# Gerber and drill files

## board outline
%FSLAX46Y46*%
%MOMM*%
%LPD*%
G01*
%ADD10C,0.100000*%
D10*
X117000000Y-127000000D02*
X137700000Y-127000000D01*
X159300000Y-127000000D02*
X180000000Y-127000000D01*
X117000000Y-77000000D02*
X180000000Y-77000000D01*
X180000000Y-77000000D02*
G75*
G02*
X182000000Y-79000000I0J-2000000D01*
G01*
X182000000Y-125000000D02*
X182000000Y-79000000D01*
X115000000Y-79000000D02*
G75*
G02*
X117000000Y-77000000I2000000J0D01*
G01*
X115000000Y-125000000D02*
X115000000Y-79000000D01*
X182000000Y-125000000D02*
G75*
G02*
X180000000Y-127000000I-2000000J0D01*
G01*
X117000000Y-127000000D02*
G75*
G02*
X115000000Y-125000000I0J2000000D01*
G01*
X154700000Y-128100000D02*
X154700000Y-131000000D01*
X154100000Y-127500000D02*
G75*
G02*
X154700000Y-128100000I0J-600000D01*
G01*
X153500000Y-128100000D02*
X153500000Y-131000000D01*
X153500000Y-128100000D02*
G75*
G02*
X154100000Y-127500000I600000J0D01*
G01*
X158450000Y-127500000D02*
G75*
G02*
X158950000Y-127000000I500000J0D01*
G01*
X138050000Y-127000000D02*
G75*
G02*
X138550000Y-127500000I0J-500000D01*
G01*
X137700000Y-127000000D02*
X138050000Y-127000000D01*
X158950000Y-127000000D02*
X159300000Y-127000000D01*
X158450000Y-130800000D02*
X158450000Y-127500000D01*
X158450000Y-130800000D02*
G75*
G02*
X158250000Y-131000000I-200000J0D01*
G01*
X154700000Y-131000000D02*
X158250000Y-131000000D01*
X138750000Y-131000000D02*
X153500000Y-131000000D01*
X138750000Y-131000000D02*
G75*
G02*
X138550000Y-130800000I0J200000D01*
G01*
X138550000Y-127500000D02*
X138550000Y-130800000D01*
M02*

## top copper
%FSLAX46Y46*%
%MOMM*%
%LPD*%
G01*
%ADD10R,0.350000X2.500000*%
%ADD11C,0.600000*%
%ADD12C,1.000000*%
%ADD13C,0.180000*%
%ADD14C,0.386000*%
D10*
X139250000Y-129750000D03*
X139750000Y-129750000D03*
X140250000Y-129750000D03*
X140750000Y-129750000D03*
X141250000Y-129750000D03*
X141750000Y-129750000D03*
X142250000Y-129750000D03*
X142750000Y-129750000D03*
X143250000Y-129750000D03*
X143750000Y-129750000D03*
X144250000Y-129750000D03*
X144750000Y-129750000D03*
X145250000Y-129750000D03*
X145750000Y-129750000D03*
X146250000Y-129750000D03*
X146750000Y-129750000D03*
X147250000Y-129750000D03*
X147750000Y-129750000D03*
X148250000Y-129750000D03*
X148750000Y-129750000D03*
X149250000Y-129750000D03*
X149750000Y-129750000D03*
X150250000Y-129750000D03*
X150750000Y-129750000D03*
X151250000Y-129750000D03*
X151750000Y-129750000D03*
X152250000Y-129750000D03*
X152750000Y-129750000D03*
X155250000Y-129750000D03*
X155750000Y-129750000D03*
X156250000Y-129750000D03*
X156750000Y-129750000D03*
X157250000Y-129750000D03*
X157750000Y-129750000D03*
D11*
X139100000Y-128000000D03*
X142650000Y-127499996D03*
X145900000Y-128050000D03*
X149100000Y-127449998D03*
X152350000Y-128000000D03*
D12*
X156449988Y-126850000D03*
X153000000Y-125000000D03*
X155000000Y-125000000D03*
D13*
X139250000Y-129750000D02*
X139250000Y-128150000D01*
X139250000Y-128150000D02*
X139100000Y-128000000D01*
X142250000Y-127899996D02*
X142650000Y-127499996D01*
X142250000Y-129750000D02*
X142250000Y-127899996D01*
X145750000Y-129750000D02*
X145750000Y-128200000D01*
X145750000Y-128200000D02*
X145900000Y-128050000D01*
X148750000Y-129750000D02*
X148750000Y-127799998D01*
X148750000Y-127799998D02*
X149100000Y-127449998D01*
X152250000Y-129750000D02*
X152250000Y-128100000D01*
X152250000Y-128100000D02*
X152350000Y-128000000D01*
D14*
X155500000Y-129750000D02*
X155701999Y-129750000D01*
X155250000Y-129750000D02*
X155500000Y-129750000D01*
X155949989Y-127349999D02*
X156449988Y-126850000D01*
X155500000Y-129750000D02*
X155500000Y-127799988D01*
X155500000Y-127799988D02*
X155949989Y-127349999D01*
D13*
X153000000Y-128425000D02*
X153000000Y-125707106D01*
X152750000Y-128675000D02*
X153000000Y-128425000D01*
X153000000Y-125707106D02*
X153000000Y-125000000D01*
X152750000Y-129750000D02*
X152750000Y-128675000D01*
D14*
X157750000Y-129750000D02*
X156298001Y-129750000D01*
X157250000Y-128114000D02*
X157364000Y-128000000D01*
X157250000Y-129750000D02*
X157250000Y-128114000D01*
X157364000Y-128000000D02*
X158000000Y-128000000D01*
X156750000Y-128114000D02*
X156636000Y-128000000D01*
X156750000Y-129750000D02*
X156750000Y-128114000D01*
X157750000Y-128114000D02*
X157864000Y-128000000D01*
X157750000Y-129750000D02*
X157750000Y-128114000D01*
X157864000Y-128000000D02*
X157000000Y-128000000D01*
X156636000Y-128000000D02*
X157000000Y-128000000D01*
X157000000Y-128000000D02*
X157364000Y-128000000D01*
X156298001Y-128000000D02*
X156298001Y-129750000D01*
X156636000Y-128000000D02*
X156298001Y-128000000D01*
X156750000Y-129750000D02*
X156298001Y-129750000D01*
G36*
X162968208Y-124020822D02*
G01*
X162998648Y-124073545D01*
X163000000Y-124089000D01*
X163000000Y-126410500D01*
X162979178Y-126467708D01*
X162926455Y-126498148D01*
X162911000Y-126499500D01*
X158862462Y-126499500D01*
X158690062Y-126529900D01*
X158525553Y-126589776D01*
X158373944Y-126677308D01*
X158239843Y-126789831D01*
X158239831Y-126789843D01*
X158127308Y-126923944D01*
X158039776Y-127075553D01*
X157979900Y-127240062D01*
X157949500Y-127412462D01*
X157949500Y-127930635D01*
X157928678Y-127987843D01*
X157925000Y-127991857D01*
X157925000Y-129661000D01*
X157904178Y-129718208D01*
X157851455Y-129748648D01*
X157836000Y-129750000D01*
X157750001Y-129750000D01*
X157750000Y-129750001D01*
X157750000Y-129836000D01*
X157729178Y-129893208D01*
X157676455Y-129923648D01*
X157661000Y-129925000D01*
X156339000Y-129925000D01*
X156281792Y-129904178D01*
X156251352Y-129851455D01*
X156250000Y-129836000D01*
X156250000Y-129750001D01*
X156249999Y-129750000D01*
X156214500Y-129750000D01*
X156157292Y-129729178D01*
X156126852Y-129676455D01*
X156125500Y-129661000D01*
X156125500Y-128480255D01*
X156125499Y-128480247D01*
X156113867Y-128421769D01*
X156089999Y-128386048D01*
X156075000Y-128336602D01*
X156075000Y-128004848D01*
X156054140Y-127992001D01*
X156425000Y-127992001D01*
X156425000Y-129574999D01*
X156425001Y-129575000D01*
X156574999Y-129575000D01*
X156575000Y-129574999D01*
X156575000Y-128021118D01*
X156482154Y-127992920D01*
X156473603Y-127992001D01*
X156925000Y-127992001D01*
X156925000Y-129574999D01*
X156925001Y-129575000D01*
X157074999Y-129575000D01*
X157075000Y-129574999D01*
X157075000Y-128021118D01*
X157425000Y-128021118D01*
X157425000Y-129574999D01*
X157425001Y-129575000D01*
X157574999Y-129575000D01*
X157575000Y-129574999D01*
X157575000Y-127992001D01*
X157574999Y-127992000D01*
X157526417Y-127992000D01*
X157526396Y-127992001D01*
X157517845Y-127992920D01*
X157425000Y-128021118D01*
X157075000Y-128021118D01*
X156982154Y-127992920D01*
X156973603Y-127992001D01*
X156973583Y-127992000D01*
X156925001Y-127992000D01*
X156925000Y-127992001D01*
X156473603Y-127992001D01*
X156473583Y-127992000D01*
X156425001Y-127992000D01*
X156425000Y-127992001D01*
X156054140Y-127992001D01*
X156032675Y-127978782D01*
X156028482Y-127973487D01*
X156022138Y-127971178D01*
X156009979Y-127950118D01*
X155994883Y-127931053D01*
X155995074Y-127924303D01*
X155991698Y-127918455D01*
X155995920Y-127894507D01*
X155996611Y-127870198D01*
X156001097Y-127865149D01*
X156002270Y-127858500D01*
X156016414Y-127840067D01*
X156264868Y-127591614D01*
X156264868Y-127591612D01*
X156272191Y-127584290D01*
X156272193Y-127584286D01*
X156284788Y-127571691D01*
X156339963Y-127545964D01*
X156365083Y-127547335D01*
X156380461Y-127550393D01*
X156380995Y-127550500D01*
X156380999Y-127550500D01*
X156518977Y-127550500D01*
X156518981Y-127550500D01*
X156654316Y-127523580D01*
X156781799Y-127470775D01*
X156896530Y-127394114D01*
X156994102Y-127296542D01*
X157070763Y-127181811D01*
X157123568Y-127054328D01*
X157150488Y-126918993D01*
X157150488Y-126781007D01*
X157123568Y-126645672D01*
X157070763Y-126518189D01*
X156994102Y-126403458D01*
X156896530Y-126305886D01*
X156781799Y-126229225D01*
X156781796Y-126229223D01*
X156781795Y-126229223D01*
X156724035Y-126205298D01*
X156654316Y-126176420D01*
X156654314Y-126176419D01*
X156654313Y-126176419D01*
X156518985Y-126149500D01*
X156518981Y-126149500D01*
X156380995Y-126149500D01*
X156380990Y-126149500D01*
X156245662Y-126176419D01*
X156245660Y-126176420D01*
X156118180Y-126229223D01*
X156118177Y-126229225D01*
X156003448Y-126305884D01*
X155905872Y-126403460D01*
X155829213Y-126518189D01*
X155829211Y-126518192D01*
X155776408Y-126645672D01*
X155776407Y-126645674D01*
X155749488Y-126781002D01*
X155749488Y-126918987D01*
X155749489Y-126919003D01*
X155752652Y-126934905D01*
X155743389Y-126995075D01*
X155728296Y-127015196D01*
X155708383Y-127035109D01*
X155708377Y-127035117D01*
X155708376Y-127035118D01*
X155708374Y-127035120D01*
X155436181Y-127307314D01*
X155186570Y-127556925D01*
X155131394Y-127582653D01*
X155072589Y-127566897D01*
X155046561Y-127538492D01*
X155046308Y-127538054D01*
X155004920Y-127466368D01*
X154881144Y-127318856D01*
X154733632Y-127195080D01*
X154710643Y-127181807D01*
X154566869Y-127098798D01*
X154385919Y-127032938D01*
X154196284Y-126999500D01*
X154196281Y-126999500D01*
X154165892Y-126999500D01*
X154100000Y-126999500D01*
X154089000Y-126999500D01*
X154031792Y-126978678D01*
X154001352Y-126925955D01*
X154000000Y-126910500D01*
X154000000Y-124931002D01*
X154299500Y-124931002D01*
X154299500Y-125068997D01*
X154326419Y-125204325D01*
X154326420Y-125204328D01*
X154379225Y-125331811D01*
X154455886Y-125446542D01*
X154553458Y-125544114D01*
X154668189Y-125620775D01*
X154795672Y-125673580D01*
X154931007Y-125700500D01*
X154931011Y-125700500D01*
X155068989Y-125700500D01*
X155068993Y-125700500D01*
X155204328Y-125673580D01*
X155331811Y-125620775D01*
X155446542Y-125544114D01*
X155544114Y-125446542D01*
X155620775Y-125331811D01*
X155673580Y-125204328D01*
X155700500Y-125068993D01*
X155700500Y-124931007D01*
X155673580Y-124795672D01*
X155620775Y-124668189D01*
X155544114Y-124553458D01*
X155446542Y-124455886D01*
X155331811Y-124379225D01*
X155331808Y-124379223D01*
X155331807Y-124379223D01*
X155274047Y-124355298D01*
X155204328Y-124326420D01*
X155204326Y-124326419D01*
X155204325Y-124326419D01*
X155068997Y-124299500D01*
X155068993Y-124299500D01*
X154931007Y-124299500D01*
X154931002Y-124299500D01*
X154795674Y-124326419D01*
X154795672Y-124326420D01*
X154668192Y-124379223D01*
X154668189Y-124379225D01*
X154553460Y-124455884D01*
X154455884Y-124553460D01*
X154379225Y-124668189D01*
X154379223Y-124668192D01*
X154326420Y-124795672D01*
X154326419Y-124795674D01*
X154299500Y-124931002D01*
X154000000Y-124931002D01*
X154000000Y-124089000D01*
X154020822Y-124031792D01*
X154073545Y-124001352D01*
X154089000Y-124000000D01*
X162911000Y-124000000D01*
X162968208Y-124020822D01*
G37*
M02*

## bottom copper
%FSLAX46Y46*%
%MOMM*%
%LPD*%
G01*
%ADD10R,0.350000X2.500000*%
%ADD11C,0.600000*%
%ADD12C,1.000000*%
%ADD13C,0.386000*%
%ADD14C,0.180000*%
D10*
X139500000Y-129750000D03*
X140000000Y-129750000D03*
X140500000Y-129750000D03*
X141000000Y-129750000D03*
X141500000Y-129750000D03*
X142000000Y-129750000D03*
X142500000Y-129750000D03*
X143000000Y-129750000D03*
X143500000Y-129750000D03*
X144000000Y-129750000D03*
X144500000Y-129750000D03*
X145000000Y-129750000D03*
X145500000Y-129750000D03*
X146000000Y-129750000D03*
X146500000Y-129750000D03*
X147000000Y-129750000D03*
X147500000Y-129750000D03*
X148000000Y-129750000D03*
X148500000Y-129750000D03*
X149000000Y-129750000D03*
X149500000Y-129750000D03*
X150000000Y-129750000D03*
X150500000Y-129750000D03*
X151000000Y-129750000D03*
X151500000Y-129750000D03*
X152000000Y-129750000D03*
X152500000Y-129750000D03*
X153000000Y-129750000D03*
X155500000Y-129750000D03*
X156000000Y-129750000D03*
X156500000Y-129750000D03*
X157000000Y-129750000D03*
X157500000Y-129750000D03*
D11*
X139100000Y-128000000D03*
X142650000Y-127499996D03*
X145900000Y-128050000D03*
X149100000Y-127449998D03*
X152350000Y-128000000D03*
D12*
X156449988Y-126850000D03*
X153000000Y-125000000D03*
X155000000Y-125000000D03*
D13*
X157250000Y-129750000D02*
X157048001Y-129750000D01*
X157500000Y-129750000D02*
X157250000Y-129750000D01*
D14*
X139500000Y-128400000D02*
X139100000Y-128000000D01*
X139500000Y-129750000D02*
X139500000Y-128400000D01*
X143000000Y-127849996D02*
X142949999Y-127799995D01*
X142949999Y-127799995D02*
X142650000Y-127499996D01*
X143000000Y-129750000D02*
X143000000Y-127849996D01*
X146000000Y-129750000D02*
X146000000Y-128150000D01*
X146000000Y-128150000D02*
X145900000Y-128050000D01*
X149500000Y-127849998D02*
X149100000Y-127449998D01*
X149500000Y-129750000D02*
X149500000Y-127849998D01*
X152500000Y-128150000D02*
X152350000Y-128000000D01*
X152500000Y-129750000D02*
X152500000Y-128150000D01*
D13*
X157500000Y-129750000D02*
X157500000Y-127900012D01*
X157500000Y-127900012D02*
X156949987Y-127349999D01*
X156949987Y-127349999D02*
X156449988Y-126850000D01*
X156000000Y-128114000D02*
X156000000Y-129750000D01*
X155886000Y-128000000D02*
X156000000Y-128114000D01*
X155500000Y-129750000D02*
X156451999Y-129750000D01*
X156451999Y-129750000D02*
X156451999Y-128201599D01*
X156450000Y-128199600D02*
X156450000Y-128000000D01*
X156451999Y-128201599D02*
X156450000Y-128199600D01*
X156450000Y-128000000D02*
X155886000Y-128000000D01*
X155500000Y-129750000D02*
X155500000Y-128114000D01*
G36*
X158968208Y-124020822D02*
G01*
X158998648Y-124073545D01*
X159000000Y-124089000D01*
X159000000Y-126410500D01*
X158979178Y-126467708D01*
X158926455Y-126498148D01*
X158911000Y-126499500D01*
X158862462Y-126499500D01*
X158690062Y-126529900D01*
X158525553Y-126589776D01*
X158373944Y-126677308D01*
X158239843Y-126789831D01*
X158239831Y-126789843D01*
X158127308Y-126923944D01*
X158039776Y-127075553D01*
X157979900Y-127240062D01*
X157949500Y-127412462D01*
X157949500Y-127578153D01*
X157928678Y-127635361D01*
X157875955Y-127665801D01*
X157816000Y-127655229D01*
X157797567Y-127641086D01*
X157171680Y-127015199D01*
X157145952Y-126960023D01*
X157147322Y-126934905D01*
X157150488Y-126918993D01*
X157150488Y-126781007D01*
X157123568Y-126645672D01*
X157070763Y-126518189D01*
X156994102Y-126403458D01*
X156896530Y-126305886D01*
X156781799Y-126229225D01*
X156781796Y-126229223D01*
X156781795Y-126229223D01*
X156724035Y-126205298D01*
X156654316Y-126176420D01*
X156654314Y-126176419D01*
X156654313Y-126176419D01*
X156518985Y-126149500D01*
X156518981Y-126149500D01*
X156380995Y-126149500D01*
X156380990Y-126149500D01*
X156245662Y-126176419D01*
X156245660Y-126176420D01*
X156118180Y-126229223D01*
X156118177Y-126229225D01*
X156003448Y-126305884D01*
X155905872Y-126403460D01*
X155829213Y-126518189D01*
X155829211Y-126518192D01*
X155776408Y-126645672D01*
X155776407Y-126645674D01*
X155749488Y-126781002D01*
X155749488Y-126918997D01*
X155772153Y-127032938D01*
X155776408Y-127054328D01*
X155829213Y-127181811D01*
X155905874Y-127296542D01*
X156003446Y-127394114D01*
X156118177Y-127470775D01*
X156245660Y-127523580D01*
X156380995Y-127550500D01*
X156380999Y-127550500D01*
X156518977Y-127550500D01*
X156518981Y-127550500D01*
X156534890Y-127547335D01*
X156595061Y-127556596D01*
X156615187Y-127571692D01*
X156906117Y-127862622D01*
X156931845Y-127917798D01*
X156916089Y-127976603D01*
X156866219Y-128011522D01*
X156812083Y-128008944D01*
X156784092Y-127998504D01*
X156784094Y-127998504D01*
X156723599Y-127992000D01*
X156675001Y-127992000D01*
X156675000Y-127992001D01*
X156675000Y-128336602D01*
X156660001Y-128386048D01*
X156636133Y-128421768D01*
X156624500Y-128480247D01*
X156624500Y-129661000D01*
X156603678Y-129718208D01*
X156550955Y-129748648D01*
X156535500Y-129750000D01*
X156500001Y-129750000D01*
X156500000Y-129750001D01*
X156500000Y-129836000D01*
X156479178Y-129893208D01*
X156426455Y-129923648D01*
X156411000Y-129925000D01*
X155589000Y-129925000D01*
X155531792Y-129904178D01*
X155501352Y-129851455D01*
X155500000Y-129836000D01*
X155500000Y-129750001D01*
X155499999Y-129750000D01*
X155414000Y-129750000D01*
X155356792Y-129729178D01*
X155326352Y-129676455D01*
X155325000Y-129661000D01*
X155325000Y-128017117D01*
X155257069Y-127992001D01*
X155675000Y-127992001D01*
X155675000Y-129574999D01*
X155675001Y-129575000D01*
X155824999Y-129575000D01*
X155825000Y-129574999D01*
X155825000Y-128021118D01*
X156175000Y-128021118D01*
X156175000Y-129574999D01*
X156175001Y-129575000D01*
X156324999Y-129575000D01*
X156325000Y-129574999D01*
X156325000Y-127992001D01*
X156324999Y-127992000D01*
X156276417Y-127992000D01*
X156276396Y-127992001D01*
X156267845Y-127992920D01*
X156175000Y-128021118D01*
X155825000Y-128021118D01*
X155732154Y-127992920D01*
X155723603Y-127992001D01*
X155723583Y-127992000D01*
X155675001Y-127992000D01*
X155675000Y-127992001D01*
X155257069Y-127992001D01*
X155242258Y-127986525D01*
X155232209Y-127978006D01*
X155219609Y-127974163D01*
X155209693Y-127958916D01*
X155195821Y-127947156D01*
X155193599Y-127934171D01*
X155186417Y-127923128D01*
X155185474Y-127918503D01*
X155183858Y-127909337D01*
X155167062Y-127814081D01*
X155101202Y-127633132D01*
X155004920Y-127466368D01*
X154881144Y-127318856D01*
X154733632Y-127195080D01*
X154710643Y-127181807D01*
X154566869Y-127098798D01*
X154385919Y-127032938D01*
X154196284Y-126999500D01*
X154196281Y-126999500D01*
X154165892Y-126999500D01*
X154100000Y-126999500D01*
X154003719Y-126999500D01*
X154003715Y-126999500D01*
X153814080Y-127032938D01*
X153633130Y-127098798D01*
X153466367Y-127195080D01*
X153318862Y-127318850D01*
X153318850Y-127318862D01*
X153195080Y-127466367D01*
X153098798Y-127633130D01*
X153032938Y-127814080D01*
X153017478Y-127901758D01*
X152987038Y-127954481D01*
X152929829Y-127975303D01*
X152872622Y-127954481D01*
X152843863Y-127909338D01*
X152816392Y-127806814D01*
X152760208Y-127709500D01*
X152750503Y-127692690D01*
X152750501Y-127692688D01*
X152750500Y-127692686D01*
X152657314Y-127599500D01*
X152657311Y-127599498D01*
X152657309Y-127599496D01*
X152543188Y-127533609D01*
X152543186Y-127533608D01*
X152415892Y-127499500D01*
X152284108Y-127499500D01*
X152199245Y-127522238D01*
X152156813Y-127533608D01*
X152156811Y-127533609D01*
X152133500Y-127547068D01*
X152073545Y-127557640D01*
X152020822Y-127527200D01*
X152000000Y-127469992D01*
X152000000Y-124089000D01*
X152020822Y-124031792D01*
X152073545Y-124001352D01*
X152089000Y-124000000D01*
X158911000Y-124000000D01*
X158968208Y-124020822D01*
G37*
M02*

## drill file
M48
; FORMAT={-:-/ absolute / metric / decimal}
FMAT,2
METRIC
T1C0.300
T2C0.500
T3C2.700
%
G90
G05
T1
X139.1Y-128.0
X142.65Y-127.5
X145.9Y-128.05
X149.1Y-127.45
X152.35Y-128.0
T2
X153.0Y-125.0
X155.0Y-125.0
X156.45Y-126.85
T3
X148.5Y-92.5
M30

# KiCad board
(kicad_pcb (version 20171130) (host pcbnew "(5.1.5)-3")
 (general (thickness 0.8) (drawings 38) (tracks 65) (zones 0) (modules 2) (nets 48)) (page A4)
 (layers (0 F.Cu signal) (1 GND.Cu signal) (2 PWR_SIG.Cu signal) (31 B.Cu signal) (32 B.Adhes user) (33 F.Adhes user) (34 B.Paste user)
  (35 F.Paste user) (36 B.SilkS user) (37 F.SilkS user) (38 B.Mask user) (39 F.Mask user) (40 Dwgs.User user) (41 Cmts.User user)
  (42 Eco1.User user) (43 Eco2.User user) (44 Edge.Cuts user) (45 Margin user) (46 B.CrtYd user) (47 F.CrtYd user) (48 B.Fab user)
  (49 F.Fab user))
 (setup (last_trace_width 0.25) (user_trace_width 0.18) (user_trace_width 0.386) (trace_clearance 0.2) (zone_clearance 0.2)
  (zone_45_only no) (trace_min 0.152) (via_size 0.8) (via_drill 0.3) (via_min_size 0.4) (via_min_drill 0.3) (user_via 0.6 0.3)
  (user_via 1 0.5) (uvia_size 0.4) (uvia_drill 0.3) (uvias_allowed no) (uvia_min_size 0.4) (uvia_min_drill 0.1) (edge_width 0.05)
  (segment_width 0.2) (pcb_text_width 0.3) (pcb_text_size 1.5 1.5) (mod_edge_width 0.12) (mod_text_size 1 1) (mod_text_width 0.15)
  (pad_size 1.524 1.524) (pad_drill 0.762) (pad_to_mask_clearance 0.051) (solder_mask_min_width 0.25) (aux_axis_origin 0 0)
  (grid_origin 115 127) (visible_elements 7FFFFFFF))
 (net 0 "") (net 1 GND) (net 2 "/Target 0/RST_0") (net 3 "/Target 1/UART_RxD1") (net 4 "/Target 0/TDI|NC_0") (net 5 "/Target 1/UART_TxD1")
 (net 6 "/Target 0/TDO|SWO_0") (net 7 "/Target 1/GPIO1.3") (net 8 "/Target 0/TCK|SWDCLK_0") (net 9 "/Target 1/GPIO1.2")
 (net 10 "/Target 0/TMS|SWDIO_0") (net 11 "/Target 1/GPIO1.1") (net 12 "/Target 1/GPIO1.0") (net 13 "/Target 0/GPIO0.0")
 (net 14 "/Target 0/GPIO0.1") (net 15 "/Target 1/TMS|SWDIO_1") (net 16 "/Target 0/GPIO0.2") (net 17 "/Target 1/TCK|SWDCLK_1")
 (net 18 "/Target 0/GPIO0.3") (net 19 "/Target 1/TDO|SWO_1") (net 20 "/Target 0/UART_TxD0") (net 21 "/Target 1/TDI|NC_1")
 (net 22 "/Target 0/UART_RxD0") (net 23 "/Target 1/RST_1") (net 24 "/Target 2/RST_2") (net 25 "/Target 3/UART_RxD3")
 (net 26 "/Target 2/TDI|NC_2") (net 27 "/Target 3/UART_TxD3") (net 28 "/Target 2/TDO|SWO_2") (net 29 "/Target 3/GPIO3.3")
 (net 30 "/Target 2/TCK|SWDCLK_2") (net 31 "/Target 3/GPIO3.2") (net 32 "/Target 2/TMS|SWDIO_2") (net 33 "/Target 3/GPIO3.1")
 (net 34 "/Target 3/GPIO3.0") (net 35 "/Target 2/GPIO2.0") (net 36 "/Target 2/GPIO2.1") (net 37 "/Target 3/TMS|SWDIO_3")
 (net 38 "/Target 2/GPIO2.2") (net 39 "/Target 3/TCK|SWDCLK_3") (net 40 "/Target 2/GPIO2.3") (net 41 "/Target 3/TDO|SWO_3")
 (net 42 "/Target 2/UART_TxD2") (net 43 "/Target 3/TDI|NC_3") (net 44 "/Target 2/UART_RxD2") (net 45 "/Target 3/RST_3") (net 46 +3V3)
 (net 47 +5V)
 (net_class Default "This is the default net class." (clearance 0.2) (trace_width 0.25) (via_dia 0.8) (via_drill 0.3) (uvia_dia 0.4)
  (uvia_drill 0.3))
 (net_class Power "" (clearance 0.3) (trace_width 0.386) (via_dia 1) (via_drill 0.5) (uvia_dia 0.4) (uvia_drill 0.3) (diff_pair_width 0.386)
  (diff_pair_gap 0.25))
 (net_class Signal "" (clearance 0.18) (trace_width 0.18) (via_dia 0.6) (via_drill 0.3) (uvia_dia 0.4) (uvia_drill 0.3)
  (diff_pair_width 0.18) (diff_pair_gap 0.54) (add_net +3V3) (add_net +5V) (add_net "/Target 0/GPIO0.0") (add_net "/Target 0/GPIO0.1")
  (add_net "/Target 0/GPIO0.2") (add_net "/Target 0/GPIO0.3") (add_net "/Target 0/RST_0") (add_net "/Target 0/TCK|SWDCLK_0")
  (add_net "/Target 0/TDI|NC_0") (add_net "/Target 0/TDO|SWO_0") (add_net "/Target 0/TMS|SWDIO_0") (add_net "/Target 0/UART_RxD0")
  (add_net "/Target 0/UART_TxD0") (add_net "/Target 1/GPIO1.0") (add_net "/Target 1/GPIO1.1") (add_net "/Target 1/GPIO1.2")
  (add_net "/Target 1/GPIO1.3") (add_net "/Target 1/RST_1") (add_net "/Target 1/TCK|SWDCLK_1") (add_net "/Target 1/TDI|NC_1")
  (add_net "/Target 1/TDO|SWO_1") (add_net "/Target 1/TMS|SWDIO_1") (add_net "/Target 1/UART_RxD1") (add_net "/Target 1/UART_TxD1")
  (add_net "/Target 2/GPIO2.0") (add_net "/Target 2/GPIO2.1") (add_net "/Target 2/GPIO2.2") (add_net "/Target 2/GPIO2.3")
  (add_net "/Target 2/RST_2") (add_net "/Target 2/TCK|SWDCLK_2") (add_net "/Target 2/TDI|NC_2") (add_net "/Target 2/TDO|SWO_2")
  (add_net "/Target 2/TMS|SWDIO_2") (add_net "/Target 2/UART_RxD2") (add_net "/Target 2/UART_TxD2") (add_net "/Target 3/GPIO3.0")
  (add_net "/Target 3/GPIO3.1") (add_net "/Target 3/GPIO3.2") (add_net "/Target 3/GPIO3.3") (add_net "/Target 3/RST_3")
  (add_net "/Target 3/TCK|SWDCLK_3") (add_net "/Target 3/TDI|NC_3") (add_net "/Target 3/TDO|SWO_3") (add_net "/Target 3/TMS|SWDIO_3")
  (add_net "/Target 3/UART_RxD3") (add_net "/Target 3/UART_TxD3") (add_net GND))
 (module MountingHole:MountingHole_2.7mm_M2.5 (layer F.Cu) (at 148.5 92.5)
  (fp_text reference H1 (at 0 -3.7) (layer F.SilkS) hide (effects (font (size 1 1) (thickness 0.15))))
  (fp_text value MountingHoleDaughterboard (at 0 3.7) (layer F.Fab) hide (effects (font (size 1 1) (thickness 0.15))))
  (pad 1 np_thru_hole circle (at 0 0) (size 2.7 2.7) (drill 2.7) (layers *.Cu *.Mask)))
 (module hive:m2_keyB (layer F.Cu) (at 148.5 131)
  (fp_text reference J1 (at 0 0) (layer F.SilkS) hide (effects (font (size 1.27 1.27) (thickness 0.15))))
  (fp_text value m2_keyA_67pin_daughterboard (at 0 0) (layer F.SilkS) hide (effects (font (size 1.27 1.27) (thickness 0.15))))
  (fp_line (start 6.2 -2.9) (end 6.2 0) (layer Edge.Cuts) (width 0.1))
  (fp_arc (start 5.6 -2.9) (end 5.6 -3.5) (angle 90) (layer Edge.Cuts) (width 0.1))
  (fp_line (start 5 -2.9) (end 5 0) (layer Edge.Cuts) (width 0.1))
  (fp_arc (start 5.6 -2.9) (end 5.6 -3.5) (angle -90) (layer Edge.Cuts) (width 0.1))
  (fp_arc (start 10.45 -3.5) (end 9.95 -3.5) (angle 90) (layer Edge.Cuts) (width 0.1))
  (fp_arc (start -10.45 -3.5) (end -10.45 -4) (angle 90) (layer Edge.Cuts) (width 0.1))
  (fp_line (start -10.8 -4) (end -10.45 -4) (layer Edge.Cuts) (width 0.1))
  (fp_line (start 10.45 -4) (end 10.8 -4) (layer Edge.Cuts) (width 0.1))
  (fp_line (start 9.95 -0.2) (end 9.95 -3.5) (layer Edge.Cuts) (width 0.1))
  (fp_arc (start 9.75 -0.2) (end 9.75 0) (angle -90) (layer Edge.Cuts) (width 0.1))
  (fp_line (start 6.2 0) (end 9.75 0) (layer Edge.Cuts) (width 0.1))
  (fp_line (start -9.75 0) (end 5 0) (layer Edge.Cuts) (width 0.1))
  (fp_arc (start -9.75 -0.2) (end -9.95 -0.2) (angle -90) (layer Edge.Cuts) (width 0.1))
  (fp_line (start -9.95 -3.5) (end -9.95 -0.2) (layer Edge.Cuts) (width 0.1))
  (pad 75 smd rect (at -9.25 -1.25) (size 0.35 2.5) (layers F.Cu F.Paste F.Mask) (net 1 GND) (solder_mask_margin 0.1016))
  (pad 74 smd rect (at -9 -1.25) (size 0.35 2.5) (layers B.Cu B.Paste B.Mask) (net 1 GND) (solder_mask_margin 0.1016))
  (pad 73 smd rect (at -8.75 -1.25) (size 0.35 2.5) (layers F.Cu F.Paste F.Mask) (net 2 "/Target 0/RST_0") (solder_mask_margin 0.1016))
  (pad 72 smd rect (at -8.5 -1.25) (size 0.35 2.5) (layers B.Cu B.Paste B.Mask) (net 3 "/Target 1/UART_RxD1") (solder_mask_margin 0.1016))
  (pad 71 smd rect (at -8.25 -1.25) (size 0.35 2.5) (layers F.Cu F.Paste F.Mask) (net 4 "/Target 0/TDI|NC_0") (solder_mask_margin 0.1016))
  (pad 70 smd rect (at -8 -1.25) (size 0.35 2.5) (layers B.Cu B.Paste B.Mask) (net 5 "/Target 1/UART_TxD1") (solder_mask_margin 0.1016))
  (pad 69 smd rect (at -7.75 -1.25) (size 0.35 2.5) (layers F.Cu F.Paste F.Mask) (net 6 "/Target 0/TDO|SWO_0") (solder_mask_margin 0.1016))
  (pad 68 smd rect (at -7.5 -1.25) (size 0.35 2.5) (layers B.Cu B.Paste B.Mask) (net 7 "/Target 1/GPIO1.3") (solder_mask_margin 0.1016))
  (pad 67 smd rect (at -7.25 -1.25) (size 0.35 2.5) (layers F.Cu F.Paste F.Mask) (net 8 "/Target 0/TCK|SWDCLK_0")
   (solder_mask_margin 0.1016))
  (pad 66 smd rect (at -7 -1.25) (size 0.35 2.5) (layers B.Cu B.Paste B.Mask) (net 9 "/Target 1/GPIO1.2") (solder_mask_margin 0.1016))
  (pad 65 smd rect (at -6.75 -1.25) (size 0.35 2.5) (layers F.Cu F.Paste F.Mask) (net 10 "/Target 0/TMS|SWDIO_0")
   (solder_mask_margin 0.1016))
  (pad 64 smd rect (at -6.5 -1.25) (size 0.35 2.5) (layers B.Cu B.Paste B.Mask) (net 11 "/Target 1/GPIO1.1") (solder_mask_margin 0.1016))
  (pad 63 smd rect (at -6.25 -1.25) (size 0.35 2.5) (layers F.Cu F.Paste F.Mask) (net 1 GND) (solder_mask_margin 0.1016))
  (pad 62 smd rect (at -6 -1.25) (size 0.35 2.5) (layers B.Cu B.Paste B.Mask) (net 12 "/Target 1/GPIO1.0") (solder_mask_margin 0.1016))
  (pad 61 smd rect (at -5.75 -1.25) (size 0.35 2.5) (layers F.Cu F.Paste F.Mask) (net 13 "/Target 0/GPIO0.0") (solder_mask_margin 0.1016))
  (pad 60 smd rect (at -5.5 -1.25) (size 0.35 2.5) (layers B.Cu B.Paste B.Mask) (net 1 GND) (solder_mask_margin 0.1016))
  (pad 59 smd rect (at -5.25 -1.25) (size 0.35 2.5) (layers F.Cu F.Paste F.Mask) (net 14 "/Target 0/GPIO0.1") (solder_mask_margin 0.1016))
  (pad 58 smd rect (at -5 -1.25) (size 0.35 2.5) (layers B.Cu B.Paste B.Mask) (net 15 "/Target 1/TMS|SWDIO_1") (solder_mask_margin 0.1016))
  (pad 57 smd rect (at -4.75 -1.25) (size 0.35 2.5) (layers F.Cu F.Paste F.Mask) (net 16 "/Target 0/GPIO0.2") (solder_mask_margin 0.1016))
  (pad 56 smd rect (at -4.5 -1.25) (size 0.35 2.5) (layers B.Cu B.Paste B.Mask) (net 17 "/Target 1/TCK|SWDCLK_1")
   (solder_mask_margin 0.1016))
  (pad 55 smd rect (at -4.25 -1.25) (size 0.35 2.5) (layers F.Cu F.Paste F.Mask) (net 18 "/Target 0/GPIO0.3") (solder_mask_margin 0.1016))
  (pad 54 smd rect (at -4 -1.25) (size 0.35 2.5) (layers B.Cu B.Paste B.Mask) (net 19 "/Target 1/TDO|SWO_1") (solder_mask_margin 0.1016))
  (pad 53 smd rect (at -3.75 -1.25) (size 0.35 2.5) (layers F.Cu F.Paste F.Mask) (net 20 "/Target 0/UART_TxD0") (solder_mask_margin 0.1016))
  (pad 52 smd rect (at -3.5 -1.25) (size 0.35 2.5) (layers B.Cu B.Paste B.Mask) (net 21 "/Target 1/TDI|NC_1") (solder_mask_margin 0.1016))
  (pad 51 smd rect (at -3.25 -1.25) (size 0.35 2.5) (layers F.Cu F.Paste F.Mask) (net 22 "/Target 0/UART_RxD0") (solder_mask_margin 0.1016))
  (pad 50 smd rect (at -3 -1.25) (size 0.35 2.5) (layers B.Cu B.Paste B.Mask) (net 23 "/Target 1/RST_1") (solder_mask_margin 0.1016))
  (pad 49 smd rect (at -2.75 -1.25) (size 0.35 2.5) (layers F.Cu F.Paste F.Mask) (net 1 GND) (solder_mask_margin 0.1016))
  (pad 48 smd rect (at -2.5 -1.25) (size 0.35 2.5) (layers B.Cu B.Paste B.Mask) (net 1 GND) (solder_mask_margin 0.1016))
  (pad 47 smd rect (at -2.25 -1.25) (size 0.35 2.5) (layers F.Cu F.Paste F.Mask) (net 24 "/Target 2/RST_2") (solder_mask_margin 0.1016))
  (pad 46 smd rect (at -2 -1.25) (size 0.35 2.5) (layers B.Cu B.Paste B.Mask) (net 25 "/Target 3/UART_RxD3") (solder_mask_margin 0.1016))
  (pad 45 smd rect (at -1.75 -1.25) (size 0.35 2.5) (layers F.Cu F.Paste F.Mask) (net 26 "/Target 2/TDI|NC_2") (solder_mask_margin 0.1016))
  (pad 44 smd rect (at -1.5 -1.25) (size 0.35 2.5) (layers B.Cu B.Paste B.Mask) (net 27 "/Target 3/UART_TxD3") (solder_mask_margin 0.1016))
  (pad 43 smd rect (at -1.25 -1.25) (size 0.35 2.5) (layers F.Cu F.Paste F.Mask) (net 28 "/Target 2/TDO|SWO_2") (solder_mask_margin 0.1016))
  (pad 42 smd rect (at -1 -1.25) (size 0.35 2.5) (layers B.Cu B.Paste B.Mask) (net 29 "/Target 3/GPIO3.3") (solder_mask_margin 0.1016))
  (pad 41 smd rect (at -0.75 -1.25) (size 0.35 2.5) (layers F.Cu F.Paste F.Mask) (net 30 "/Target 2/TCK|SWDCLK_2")
   (solder_mask_margin 0.1016))
  (pad 40 smd rect (at -0.5 -1.25) (size 0.35 2.5) (layers B.Cu B.Paste B.Mask) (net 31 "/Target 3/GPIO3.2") (solder_mask_margin 0.1016))
  (pad 39 smd rect (at -0.25 -1.25) (size 0.35 2.5) (layers F.Cu F.Paste F.Mask) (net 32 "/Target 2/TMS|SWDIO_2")
   (solder_mask_margin 0.1016))
  (pad 38 smd rect (at 0 -1.25) (size 0.35 2.5) (layers B.Cu B.Paste B.Mask) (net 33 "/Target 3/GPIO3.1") (solder_mask_margin 0.1016))
  (pad 37 smd rect (at 0.25 -1.25) (size 0.35 2.5) (layers F.Cu F.Paste F.Mask) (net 1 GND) (solder_mask_margin 0.1016))
  (pad 36 smd rect (at 0.5 -1.25) (size 0.35 2.5) (layers B.Cu B.Paste B.Mask) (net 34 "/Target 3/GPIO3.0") (solder_mask_margin 0.1016))
  (pad 35 smd rect (at 0.75 -1.25) (size 0.35 2.5) (layers F.Cu F.Paste F.Mask) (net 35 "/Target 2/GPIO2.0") (solder_mask_margin 0.1016))
  (pad 34 smd rect (at 1 -1.25) (size 0.35 2.5) (layers B.Cu B.Paste B.Mask) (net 1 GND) (solder_mask_margin 0.1016))
  (pad 33 smd rect (at 1.25 -1.25) (size 0.35 2.5) (layers F.Cu F.Paste F.Mask) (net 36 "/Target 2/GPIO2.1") (solder_mask_margin 0.1016))
  (pad 32 smd rect (at 1.5 -1.25) (size 0.35 2.5) (layers B.Cu B.Paste B.Mask) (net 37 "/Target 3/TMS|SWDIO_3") (solder_mask_margin 0.1016))
  (pad 31 smd rect (at 1.75 -1.25) (size 0.35 2.5) (layers F.Cu F.Paste F.Mask) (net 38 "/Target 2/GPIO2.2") (solder_mask_margin 0.1016))
  (pad 30 smd rect (at 2 -1.25) (size 0.35 2.5) (layers B.Cu B.Paste B.Mask) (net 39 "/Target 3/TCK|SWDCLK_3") (solder_mask_margin 0.1016))
  (pad 29 smd rect (at 2.25 -1.25) (size 0.35 2.5) (layers F.Cu F.Paste F.Mask) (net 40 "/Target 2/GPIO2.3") (solder_mask_margin 0.1016))
  (pad 28 smd rect (at 2.5 -1.25) (size 0.35 2.5) (layers B.Cu B.Paste B.Mask) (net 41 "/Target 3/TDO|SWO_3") (solder_mask_margin 0.1016))
  (pad 27 smd rect (at 2.75 -1.25) (size 0.35 2.5) (layers F.Cu F.Paste F.Mask) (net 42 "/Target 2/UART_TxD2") (solder_mask_margin 0.1016))
  (pad 26 smd rect (at 3 -1.25) (size 0.35 2.5) (layers B.Cu B.Paste B.Mask) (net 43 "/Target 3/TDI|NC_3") (solder_mask_margin 0.1016))
  (pad 25 smd rect (at 3.25 -1.25) (size 0.35 2.5) (layers F.Cu F.Paste F.Mask) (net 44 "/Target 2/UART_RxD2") (solder_mask_margin 0.1016))
  (pad 24 smd rect (at 3.5 -1.25) (size 0.35 2.5) (layers B.Cu B.Paste B.Mask) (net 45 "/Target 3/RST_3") (solder_mask_margin 0.1016))
  (pad 23 smd rect (at 3.75 -1.25) (size 0.35 2.5) (layers F.Cu F.Paste F.Mask) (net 1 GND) (solder_mask_margin 0.1016))
  (pad 22 smd rect (at 4 -1.25) (size 0.35 2.5) (layers B.Cu B.Paste B.Mask) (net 1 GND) (solder_mask_margin 0.1016))
  (pad 21 smd rect (at 4.25 -1.25) (size 0.35 2.5) (layers F.Cu F.Paste F.Mask) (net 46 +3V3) (solder_mask_margin 0.1016))
  (pad 20 smd rect (at 4.5 -1.25) (size 0.35 2.5) (layers B.Cu B.Paste B.Mask) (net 46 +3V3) (solder_mask_margin 0.1016))
  (pad 11 smd rect (at 6.75 -1.25) (size 0.35 2.5) (layers F.Cu F.Paste F.Mask) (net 1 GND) (solder_mask_margin 0.1016))
  (pad 10 smd rect (at 7 -1.25) (size 0.35 2.5) (layers B.Cu B.Paste B.Mask) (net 46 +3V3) (solder_mask_margin 0.1016))
  (pad 9 smd rect (at 7.25 -1.25) (size 0.35 2.5) (layers F.Cu F.Paste F.Mask) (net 1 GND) (solder_mask_margin 0.1016))
  (pad 8 smd rect (at 7.5 -1.25) (size 0.35 2.5) (layers B.Cu B.Paste B.Mask) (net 46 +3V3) (solder_mask_margin 0.1016))
  (pad 7 smd rect (at 7.75 -1.25) (size 0.35 2.5) (layers F.Cu F.Paste F.Mask) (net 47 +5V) (solder_mask_margin 0.1016))
  (pad 6 smd rect (at 8 -1.25) (size 0.35 2.5) (layers B.Cu B.Paste B.Mask) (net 46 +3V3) (solder_mask_margin 0.1016))
  (pad 5 smd rect (at 8.25 -1.25) (size 0.35 2.5) (layers F.Cu F.Paste F.Mask) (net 47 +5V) (solder_mask_margin 0.1016))
  (pad 4 smd rect (at 8.5 -1.25) (size 0.35 2.5) (layers B.Cu B.Paste B.Mask) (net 1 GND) (solder_mask_margin 0.1016))
  (pad 3 smd rect (at 8.75 -1.25) (size 0.35 2.5) (layers F.Cu F.Paste F.Mask) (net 47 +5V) (solder_mask_margin 0.1016))
  (pad 2 smd rect (at 9 -1.25) (size 0.35 2.5) (layers B.Cu B.Paste B.Mask) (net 1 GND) (solder_mask_margin 0.1016))
  (pad 1 smd rect (at 9.25 -1.25) (size 0.35 2.5) (layers F.Cu F.Paste F.Mask) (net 47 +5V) (solder_mask_margin 0.1016)))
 (gr_line (start 117 127) (end 137.7 127) (layer Edge.Cuts) (width 0.1))
 (gr_line (start 159.3 127) (end 180 127) (layer Edge.Cuts) (width 0.1))
 (gr_line (start 117 77) (end 180 77) (layer Edge.Cuts) (width 0.1))
 (gr_arc (start 180 79) (end 182 79) (angle -90) (layer Edge.Cuts) (width 0.1))
 (gr_line (start 182 125) (end 182 79) (layer Edge.Cuts) (width 0.1))
 (gr_arc (start 117 79) (end 117 77) (angle -90) (layer Edge.Cuts) (width 0.1))
 (gr_line (start 115 125) (end 115 79) (layer Edge.Cuts) (width 0.1))
 (gr_arc (start 180 125) (end 180 127) (angle -90) (layer Edge.Cuts) (width 0.1))
 (gr_arc (start 117 125) (end 115 125) (angle -90) (layer Edge.Cuts) (width 0.1))
 (segment (start 157.25 129.75) (end 157.048001 129.75) (width 0.386) (layer B.Cu) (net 1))
 (segment (start 157.5 129.75) (end 157.25 129.75) (width 0.386) (layer B.Cu) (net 1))
 (via (at 139.1 128) (size 0.6) (drill 0.3) (layers F.Cu B.Cu) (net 1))
 (segment (start 139.25 129.75) (end 139.25 128.15) (width 0.18) (layer F.Cu) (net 1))
 (segment (start 139.25 128.15) (end 139.1 128) (width 0.18) (layer F.Cu) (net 1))
 (segment (start 139.5 128.4) (end 139.1 128) (width 0.18) (layer B.Cu) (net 1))
 (segment (start 139.5 129.75) (end 139.5 128.4) (width 0.18) (layer B.Cu) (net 1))
 (segment (start 143 127.849996) (end 142.949999 127.799995) (width 0.18) (layer B.Cu) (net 1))
 (segment (start 142.949999 127.799995) (end 142.65 127.499996) (width 0.18) (layer B.Cu) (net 1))
 (via (at 142.65 127.499996) (size 0.6) (drill 0.3) (layers F.Cu B.Cu) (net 1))
 (segment (start 143 129.75) (end 143 127.849996) (width 0.18) (layer B.Cu) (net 1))
 (segment (start 142.25 127.899996) (end 142.65 127.499996) (width 0.18) (layer F.Cu) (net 1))
 (segment (start 142.25 129.75) (end 142.25 127.899996) (width 0.18) (layer F.Cu) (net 1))
 (via (at 145.9 128.05) (size 0.6) (drill 0.3) (layers F.Cu B.Cu) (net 1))
 (segment (start 146 129.75) (end 146 128.15) (width 0.18) (layer B.Cu) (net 1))
 (segment (start 145.75 129.75) (end 145.75 128.2) (width 0.18) (layer F.Cu) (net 1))
 (segment (start 146 128.15) (end 145.9 128.05) (width 0.18) (layer B.Cu) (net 1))
 (segment (start 145.75 128.2) (end 145.9 128.05) (width 0.18) (layer F.Cu) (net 1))
 (via (at 149.1 127.449998) (size 0.6) (drill 0.3) (layers F.Cu B.Cu) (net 1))
 (segment (start 149.5 127.849998) (end 149.1 127.449998) (width 0.18) (layer B.Cu) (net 1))
 (segment (start 148.75 129.75) (end 148.75 127.799998) (width 0.18) (layer F.Cu) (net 1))
 (segment (start 149.5 129.75) (end 149.5 127.849998) (width 0.18) (layer B.Cu) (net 1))
 (segment (start 148.75 127.799998) (end 149.1 127.449998) (width 0.18) (layer F.Cu) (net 1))
 (segment (start 152.25 129.75) (end 152.25 128.1) (width 0.18) (layer F.Cu) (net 1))
 (segment (start 152.5 128.15) (end 152.35 128) (width 0.18) (layer B.Cu) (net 1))
 (segment (start 152.5 129.75) (end 152.5 128.15) (width 0.18) (layer B.Cu) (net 1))
 (via (at 152.35 128) (size 0.6) (drill 0.3) (layers F.Cu B.Cu) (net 1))
 (segment (start 152.25 128.1) (end 152.35 128) (width 0.18) (layer F.Cu) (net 1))
 (segment (start 155.5 129.75) (end 155.701999 129.75) (width 0.386) (layer F.Cu) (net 1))
 (segment (start 155.25 129.75) (end 155.5 129.75) (width 0.386) (layer F.Cu) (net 1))
 (via (at 156.449988 126.85) (size 1) (drill 0.5) (layers F.Cu B.Cu) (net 1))
 (segment (start 157.5 129.75) (end 157.5 127.900012) (width 0.386) (layer B.Cu) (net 1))
 (segment (start 157.5 127.900012) (end 156.949987 127.349999) (width 0.386) (layer B.Cu) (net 1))
 (segment (start 156.949987 127.349999) (end 156.449988 126.85) (width 0.386) (layer B.Cu) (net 1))
 (segment (start 155.949989 127.349999) (end 156.449988 126.85) (width 0.386) (layer F.Cu) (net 1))
 (segment (start 155.5 129.75) (end 155.5 127.799988) (width 0.386) (layer F.Cu) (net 1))
 (segment (start 155.5 127.799988) (end 155.949989 127.349999) (width 0.386) (layer F.Cu) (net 1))
 (via (at 153 125) (size 1) (drill 0.5) (layers F.Cu B.Cu) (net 46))
 (segment (start 156 128.114) (end 156 129.75) (width 0.386) (layer B.Cu) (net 46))
 (segment (start 155.886 128) (end 156 128.114) (width 0.386) (layer B.Cu) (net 46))
 (segment (start 155.5 129.75) (end 156.451999 129.75) (width 0.386) (layer B.Cu) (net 46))
 (segment (start 156.451999 129.75) (end 156.451999 128.201599) (width 0.386) (layer B.Cu) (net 46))
 (segment (start 156.45 128.1996) (end 156.45 128) (width 0.386) (layer B.Cu) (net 46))
 (segment (start 156.451999 128.201599) (end 156.45 128.1996) (width 0.386) (layer B.Cu) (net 46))
 (segment (start 156.45 128) (end 155.886 128) (width 0.386) (layer B.Cu) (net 46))
 (segment (start 155.5 129.75) (end 155.5 128.114) (width 0.386) (layer B.Cu) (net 46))
 (via (at 155 125) (size 1) (drill 0.5) (layers F.Cu B.Cu) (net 46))
 (segment (start 153 128.425) (end 153 125.707106) (width 0.18) (layer F.Cu) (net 46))
 (segment (start 152.75 128.675) (end 153 128.425) (width 0.18) (layer F.Cu) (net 46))
 (segment (start 153 125.707106) (end 153 125) (width 0.18) (layer F.Cu) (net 46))
 (segment (start 152.75 129.75) (end 152.75 128.675) (width 0.18) (layer F.Cu) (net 46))
 (segment (start 157.75 129.75) (end 156.298001 129.75) (width 0.386) (layer F.Cu) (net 47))
 (segment (start 157.25 128.114) (end 157.364 128) (width 0.386) (layer F.Cu) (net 47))
 (segment (start 157.25 129.75) (end 157.25 128.114) (width 0.386) (layer F.Cu) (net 47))
 (segment (start 157.364 128) (end 158 128) (width 0.386) (layer F.Cu) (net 47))
 (segment (start 156.75 128.114) (end 156.636 128) (width 0.386) (layer F.Cu) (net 47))
 (segment (start 156.75 129.75) (end 156.75 128.114) (width 0.386) (layer F.Cu) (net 47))
 (segment (start 157.75 128.114) (end 157.864 128) (width 0.386) (layer F.Cu) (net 47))
 (segment (start 157.75 129.75) (end 157.75 128.114) (width 0.386) (layer F.Cu) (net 47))
 (segment (start 157.864 128) (end 157 128) (width 0.386) (layer F.Cu) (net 47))
 (segment (start 156.636 128) (end 157 128) (width 0.386) (layer F.Cu) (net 47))
 (segment (start 157 128) (end 157.364 128) (width 0.386) (layer F.Cu) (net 47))
 (segment (start 156.298001 128) (end 156.298001 129.75) (width 0.386) (layer F.Cu) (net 47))
 (segment (start 156.636 128) (end 156.298001 128) (width 0.386) (layer F.Cu) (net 47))
 (segment (start 156.75 129.75) (end 156.298001 129.75) (width 0.386) (layer F.Cu) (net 47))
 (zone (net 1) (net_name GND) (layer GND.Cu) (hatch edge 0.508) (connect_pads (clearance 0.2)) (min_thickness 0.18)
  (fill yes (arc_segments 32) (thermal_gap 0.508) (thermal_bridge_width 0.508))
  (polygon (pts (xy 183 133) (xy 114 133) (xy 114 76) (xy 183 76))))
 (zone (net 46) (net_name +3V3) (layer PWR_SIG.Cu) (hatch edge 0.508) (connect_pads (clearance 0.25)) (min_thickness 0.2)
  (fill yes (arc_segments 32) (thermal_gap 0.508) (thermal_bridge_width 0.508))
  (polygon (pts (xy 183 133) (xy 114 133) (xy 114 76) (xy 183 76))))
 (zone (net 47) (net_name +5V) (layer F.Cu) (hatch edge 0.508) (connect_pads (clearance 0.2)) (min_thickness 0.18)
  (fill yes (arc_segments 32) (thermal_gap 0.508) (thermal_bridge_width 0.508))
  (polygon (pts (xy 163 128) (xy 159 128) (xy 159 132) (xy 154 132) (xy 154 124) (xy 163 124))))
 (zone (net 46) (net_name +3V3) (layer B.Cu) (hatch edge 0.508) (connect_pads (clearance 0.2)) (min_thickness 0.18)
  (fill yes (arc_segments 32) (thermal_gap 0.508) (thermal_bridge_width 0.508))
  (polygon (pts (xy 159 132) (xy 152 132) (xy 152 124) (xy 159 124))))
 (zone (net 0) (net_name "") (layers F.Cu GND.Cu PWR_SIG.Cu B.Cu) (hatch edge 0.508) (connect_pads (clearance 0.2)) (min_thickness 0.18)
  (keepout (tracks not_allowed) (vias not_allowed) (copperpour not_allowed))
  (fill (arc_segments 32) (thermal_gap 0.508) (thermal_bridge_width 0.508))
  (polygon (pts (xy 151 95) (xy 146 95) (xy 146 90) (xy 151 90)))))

